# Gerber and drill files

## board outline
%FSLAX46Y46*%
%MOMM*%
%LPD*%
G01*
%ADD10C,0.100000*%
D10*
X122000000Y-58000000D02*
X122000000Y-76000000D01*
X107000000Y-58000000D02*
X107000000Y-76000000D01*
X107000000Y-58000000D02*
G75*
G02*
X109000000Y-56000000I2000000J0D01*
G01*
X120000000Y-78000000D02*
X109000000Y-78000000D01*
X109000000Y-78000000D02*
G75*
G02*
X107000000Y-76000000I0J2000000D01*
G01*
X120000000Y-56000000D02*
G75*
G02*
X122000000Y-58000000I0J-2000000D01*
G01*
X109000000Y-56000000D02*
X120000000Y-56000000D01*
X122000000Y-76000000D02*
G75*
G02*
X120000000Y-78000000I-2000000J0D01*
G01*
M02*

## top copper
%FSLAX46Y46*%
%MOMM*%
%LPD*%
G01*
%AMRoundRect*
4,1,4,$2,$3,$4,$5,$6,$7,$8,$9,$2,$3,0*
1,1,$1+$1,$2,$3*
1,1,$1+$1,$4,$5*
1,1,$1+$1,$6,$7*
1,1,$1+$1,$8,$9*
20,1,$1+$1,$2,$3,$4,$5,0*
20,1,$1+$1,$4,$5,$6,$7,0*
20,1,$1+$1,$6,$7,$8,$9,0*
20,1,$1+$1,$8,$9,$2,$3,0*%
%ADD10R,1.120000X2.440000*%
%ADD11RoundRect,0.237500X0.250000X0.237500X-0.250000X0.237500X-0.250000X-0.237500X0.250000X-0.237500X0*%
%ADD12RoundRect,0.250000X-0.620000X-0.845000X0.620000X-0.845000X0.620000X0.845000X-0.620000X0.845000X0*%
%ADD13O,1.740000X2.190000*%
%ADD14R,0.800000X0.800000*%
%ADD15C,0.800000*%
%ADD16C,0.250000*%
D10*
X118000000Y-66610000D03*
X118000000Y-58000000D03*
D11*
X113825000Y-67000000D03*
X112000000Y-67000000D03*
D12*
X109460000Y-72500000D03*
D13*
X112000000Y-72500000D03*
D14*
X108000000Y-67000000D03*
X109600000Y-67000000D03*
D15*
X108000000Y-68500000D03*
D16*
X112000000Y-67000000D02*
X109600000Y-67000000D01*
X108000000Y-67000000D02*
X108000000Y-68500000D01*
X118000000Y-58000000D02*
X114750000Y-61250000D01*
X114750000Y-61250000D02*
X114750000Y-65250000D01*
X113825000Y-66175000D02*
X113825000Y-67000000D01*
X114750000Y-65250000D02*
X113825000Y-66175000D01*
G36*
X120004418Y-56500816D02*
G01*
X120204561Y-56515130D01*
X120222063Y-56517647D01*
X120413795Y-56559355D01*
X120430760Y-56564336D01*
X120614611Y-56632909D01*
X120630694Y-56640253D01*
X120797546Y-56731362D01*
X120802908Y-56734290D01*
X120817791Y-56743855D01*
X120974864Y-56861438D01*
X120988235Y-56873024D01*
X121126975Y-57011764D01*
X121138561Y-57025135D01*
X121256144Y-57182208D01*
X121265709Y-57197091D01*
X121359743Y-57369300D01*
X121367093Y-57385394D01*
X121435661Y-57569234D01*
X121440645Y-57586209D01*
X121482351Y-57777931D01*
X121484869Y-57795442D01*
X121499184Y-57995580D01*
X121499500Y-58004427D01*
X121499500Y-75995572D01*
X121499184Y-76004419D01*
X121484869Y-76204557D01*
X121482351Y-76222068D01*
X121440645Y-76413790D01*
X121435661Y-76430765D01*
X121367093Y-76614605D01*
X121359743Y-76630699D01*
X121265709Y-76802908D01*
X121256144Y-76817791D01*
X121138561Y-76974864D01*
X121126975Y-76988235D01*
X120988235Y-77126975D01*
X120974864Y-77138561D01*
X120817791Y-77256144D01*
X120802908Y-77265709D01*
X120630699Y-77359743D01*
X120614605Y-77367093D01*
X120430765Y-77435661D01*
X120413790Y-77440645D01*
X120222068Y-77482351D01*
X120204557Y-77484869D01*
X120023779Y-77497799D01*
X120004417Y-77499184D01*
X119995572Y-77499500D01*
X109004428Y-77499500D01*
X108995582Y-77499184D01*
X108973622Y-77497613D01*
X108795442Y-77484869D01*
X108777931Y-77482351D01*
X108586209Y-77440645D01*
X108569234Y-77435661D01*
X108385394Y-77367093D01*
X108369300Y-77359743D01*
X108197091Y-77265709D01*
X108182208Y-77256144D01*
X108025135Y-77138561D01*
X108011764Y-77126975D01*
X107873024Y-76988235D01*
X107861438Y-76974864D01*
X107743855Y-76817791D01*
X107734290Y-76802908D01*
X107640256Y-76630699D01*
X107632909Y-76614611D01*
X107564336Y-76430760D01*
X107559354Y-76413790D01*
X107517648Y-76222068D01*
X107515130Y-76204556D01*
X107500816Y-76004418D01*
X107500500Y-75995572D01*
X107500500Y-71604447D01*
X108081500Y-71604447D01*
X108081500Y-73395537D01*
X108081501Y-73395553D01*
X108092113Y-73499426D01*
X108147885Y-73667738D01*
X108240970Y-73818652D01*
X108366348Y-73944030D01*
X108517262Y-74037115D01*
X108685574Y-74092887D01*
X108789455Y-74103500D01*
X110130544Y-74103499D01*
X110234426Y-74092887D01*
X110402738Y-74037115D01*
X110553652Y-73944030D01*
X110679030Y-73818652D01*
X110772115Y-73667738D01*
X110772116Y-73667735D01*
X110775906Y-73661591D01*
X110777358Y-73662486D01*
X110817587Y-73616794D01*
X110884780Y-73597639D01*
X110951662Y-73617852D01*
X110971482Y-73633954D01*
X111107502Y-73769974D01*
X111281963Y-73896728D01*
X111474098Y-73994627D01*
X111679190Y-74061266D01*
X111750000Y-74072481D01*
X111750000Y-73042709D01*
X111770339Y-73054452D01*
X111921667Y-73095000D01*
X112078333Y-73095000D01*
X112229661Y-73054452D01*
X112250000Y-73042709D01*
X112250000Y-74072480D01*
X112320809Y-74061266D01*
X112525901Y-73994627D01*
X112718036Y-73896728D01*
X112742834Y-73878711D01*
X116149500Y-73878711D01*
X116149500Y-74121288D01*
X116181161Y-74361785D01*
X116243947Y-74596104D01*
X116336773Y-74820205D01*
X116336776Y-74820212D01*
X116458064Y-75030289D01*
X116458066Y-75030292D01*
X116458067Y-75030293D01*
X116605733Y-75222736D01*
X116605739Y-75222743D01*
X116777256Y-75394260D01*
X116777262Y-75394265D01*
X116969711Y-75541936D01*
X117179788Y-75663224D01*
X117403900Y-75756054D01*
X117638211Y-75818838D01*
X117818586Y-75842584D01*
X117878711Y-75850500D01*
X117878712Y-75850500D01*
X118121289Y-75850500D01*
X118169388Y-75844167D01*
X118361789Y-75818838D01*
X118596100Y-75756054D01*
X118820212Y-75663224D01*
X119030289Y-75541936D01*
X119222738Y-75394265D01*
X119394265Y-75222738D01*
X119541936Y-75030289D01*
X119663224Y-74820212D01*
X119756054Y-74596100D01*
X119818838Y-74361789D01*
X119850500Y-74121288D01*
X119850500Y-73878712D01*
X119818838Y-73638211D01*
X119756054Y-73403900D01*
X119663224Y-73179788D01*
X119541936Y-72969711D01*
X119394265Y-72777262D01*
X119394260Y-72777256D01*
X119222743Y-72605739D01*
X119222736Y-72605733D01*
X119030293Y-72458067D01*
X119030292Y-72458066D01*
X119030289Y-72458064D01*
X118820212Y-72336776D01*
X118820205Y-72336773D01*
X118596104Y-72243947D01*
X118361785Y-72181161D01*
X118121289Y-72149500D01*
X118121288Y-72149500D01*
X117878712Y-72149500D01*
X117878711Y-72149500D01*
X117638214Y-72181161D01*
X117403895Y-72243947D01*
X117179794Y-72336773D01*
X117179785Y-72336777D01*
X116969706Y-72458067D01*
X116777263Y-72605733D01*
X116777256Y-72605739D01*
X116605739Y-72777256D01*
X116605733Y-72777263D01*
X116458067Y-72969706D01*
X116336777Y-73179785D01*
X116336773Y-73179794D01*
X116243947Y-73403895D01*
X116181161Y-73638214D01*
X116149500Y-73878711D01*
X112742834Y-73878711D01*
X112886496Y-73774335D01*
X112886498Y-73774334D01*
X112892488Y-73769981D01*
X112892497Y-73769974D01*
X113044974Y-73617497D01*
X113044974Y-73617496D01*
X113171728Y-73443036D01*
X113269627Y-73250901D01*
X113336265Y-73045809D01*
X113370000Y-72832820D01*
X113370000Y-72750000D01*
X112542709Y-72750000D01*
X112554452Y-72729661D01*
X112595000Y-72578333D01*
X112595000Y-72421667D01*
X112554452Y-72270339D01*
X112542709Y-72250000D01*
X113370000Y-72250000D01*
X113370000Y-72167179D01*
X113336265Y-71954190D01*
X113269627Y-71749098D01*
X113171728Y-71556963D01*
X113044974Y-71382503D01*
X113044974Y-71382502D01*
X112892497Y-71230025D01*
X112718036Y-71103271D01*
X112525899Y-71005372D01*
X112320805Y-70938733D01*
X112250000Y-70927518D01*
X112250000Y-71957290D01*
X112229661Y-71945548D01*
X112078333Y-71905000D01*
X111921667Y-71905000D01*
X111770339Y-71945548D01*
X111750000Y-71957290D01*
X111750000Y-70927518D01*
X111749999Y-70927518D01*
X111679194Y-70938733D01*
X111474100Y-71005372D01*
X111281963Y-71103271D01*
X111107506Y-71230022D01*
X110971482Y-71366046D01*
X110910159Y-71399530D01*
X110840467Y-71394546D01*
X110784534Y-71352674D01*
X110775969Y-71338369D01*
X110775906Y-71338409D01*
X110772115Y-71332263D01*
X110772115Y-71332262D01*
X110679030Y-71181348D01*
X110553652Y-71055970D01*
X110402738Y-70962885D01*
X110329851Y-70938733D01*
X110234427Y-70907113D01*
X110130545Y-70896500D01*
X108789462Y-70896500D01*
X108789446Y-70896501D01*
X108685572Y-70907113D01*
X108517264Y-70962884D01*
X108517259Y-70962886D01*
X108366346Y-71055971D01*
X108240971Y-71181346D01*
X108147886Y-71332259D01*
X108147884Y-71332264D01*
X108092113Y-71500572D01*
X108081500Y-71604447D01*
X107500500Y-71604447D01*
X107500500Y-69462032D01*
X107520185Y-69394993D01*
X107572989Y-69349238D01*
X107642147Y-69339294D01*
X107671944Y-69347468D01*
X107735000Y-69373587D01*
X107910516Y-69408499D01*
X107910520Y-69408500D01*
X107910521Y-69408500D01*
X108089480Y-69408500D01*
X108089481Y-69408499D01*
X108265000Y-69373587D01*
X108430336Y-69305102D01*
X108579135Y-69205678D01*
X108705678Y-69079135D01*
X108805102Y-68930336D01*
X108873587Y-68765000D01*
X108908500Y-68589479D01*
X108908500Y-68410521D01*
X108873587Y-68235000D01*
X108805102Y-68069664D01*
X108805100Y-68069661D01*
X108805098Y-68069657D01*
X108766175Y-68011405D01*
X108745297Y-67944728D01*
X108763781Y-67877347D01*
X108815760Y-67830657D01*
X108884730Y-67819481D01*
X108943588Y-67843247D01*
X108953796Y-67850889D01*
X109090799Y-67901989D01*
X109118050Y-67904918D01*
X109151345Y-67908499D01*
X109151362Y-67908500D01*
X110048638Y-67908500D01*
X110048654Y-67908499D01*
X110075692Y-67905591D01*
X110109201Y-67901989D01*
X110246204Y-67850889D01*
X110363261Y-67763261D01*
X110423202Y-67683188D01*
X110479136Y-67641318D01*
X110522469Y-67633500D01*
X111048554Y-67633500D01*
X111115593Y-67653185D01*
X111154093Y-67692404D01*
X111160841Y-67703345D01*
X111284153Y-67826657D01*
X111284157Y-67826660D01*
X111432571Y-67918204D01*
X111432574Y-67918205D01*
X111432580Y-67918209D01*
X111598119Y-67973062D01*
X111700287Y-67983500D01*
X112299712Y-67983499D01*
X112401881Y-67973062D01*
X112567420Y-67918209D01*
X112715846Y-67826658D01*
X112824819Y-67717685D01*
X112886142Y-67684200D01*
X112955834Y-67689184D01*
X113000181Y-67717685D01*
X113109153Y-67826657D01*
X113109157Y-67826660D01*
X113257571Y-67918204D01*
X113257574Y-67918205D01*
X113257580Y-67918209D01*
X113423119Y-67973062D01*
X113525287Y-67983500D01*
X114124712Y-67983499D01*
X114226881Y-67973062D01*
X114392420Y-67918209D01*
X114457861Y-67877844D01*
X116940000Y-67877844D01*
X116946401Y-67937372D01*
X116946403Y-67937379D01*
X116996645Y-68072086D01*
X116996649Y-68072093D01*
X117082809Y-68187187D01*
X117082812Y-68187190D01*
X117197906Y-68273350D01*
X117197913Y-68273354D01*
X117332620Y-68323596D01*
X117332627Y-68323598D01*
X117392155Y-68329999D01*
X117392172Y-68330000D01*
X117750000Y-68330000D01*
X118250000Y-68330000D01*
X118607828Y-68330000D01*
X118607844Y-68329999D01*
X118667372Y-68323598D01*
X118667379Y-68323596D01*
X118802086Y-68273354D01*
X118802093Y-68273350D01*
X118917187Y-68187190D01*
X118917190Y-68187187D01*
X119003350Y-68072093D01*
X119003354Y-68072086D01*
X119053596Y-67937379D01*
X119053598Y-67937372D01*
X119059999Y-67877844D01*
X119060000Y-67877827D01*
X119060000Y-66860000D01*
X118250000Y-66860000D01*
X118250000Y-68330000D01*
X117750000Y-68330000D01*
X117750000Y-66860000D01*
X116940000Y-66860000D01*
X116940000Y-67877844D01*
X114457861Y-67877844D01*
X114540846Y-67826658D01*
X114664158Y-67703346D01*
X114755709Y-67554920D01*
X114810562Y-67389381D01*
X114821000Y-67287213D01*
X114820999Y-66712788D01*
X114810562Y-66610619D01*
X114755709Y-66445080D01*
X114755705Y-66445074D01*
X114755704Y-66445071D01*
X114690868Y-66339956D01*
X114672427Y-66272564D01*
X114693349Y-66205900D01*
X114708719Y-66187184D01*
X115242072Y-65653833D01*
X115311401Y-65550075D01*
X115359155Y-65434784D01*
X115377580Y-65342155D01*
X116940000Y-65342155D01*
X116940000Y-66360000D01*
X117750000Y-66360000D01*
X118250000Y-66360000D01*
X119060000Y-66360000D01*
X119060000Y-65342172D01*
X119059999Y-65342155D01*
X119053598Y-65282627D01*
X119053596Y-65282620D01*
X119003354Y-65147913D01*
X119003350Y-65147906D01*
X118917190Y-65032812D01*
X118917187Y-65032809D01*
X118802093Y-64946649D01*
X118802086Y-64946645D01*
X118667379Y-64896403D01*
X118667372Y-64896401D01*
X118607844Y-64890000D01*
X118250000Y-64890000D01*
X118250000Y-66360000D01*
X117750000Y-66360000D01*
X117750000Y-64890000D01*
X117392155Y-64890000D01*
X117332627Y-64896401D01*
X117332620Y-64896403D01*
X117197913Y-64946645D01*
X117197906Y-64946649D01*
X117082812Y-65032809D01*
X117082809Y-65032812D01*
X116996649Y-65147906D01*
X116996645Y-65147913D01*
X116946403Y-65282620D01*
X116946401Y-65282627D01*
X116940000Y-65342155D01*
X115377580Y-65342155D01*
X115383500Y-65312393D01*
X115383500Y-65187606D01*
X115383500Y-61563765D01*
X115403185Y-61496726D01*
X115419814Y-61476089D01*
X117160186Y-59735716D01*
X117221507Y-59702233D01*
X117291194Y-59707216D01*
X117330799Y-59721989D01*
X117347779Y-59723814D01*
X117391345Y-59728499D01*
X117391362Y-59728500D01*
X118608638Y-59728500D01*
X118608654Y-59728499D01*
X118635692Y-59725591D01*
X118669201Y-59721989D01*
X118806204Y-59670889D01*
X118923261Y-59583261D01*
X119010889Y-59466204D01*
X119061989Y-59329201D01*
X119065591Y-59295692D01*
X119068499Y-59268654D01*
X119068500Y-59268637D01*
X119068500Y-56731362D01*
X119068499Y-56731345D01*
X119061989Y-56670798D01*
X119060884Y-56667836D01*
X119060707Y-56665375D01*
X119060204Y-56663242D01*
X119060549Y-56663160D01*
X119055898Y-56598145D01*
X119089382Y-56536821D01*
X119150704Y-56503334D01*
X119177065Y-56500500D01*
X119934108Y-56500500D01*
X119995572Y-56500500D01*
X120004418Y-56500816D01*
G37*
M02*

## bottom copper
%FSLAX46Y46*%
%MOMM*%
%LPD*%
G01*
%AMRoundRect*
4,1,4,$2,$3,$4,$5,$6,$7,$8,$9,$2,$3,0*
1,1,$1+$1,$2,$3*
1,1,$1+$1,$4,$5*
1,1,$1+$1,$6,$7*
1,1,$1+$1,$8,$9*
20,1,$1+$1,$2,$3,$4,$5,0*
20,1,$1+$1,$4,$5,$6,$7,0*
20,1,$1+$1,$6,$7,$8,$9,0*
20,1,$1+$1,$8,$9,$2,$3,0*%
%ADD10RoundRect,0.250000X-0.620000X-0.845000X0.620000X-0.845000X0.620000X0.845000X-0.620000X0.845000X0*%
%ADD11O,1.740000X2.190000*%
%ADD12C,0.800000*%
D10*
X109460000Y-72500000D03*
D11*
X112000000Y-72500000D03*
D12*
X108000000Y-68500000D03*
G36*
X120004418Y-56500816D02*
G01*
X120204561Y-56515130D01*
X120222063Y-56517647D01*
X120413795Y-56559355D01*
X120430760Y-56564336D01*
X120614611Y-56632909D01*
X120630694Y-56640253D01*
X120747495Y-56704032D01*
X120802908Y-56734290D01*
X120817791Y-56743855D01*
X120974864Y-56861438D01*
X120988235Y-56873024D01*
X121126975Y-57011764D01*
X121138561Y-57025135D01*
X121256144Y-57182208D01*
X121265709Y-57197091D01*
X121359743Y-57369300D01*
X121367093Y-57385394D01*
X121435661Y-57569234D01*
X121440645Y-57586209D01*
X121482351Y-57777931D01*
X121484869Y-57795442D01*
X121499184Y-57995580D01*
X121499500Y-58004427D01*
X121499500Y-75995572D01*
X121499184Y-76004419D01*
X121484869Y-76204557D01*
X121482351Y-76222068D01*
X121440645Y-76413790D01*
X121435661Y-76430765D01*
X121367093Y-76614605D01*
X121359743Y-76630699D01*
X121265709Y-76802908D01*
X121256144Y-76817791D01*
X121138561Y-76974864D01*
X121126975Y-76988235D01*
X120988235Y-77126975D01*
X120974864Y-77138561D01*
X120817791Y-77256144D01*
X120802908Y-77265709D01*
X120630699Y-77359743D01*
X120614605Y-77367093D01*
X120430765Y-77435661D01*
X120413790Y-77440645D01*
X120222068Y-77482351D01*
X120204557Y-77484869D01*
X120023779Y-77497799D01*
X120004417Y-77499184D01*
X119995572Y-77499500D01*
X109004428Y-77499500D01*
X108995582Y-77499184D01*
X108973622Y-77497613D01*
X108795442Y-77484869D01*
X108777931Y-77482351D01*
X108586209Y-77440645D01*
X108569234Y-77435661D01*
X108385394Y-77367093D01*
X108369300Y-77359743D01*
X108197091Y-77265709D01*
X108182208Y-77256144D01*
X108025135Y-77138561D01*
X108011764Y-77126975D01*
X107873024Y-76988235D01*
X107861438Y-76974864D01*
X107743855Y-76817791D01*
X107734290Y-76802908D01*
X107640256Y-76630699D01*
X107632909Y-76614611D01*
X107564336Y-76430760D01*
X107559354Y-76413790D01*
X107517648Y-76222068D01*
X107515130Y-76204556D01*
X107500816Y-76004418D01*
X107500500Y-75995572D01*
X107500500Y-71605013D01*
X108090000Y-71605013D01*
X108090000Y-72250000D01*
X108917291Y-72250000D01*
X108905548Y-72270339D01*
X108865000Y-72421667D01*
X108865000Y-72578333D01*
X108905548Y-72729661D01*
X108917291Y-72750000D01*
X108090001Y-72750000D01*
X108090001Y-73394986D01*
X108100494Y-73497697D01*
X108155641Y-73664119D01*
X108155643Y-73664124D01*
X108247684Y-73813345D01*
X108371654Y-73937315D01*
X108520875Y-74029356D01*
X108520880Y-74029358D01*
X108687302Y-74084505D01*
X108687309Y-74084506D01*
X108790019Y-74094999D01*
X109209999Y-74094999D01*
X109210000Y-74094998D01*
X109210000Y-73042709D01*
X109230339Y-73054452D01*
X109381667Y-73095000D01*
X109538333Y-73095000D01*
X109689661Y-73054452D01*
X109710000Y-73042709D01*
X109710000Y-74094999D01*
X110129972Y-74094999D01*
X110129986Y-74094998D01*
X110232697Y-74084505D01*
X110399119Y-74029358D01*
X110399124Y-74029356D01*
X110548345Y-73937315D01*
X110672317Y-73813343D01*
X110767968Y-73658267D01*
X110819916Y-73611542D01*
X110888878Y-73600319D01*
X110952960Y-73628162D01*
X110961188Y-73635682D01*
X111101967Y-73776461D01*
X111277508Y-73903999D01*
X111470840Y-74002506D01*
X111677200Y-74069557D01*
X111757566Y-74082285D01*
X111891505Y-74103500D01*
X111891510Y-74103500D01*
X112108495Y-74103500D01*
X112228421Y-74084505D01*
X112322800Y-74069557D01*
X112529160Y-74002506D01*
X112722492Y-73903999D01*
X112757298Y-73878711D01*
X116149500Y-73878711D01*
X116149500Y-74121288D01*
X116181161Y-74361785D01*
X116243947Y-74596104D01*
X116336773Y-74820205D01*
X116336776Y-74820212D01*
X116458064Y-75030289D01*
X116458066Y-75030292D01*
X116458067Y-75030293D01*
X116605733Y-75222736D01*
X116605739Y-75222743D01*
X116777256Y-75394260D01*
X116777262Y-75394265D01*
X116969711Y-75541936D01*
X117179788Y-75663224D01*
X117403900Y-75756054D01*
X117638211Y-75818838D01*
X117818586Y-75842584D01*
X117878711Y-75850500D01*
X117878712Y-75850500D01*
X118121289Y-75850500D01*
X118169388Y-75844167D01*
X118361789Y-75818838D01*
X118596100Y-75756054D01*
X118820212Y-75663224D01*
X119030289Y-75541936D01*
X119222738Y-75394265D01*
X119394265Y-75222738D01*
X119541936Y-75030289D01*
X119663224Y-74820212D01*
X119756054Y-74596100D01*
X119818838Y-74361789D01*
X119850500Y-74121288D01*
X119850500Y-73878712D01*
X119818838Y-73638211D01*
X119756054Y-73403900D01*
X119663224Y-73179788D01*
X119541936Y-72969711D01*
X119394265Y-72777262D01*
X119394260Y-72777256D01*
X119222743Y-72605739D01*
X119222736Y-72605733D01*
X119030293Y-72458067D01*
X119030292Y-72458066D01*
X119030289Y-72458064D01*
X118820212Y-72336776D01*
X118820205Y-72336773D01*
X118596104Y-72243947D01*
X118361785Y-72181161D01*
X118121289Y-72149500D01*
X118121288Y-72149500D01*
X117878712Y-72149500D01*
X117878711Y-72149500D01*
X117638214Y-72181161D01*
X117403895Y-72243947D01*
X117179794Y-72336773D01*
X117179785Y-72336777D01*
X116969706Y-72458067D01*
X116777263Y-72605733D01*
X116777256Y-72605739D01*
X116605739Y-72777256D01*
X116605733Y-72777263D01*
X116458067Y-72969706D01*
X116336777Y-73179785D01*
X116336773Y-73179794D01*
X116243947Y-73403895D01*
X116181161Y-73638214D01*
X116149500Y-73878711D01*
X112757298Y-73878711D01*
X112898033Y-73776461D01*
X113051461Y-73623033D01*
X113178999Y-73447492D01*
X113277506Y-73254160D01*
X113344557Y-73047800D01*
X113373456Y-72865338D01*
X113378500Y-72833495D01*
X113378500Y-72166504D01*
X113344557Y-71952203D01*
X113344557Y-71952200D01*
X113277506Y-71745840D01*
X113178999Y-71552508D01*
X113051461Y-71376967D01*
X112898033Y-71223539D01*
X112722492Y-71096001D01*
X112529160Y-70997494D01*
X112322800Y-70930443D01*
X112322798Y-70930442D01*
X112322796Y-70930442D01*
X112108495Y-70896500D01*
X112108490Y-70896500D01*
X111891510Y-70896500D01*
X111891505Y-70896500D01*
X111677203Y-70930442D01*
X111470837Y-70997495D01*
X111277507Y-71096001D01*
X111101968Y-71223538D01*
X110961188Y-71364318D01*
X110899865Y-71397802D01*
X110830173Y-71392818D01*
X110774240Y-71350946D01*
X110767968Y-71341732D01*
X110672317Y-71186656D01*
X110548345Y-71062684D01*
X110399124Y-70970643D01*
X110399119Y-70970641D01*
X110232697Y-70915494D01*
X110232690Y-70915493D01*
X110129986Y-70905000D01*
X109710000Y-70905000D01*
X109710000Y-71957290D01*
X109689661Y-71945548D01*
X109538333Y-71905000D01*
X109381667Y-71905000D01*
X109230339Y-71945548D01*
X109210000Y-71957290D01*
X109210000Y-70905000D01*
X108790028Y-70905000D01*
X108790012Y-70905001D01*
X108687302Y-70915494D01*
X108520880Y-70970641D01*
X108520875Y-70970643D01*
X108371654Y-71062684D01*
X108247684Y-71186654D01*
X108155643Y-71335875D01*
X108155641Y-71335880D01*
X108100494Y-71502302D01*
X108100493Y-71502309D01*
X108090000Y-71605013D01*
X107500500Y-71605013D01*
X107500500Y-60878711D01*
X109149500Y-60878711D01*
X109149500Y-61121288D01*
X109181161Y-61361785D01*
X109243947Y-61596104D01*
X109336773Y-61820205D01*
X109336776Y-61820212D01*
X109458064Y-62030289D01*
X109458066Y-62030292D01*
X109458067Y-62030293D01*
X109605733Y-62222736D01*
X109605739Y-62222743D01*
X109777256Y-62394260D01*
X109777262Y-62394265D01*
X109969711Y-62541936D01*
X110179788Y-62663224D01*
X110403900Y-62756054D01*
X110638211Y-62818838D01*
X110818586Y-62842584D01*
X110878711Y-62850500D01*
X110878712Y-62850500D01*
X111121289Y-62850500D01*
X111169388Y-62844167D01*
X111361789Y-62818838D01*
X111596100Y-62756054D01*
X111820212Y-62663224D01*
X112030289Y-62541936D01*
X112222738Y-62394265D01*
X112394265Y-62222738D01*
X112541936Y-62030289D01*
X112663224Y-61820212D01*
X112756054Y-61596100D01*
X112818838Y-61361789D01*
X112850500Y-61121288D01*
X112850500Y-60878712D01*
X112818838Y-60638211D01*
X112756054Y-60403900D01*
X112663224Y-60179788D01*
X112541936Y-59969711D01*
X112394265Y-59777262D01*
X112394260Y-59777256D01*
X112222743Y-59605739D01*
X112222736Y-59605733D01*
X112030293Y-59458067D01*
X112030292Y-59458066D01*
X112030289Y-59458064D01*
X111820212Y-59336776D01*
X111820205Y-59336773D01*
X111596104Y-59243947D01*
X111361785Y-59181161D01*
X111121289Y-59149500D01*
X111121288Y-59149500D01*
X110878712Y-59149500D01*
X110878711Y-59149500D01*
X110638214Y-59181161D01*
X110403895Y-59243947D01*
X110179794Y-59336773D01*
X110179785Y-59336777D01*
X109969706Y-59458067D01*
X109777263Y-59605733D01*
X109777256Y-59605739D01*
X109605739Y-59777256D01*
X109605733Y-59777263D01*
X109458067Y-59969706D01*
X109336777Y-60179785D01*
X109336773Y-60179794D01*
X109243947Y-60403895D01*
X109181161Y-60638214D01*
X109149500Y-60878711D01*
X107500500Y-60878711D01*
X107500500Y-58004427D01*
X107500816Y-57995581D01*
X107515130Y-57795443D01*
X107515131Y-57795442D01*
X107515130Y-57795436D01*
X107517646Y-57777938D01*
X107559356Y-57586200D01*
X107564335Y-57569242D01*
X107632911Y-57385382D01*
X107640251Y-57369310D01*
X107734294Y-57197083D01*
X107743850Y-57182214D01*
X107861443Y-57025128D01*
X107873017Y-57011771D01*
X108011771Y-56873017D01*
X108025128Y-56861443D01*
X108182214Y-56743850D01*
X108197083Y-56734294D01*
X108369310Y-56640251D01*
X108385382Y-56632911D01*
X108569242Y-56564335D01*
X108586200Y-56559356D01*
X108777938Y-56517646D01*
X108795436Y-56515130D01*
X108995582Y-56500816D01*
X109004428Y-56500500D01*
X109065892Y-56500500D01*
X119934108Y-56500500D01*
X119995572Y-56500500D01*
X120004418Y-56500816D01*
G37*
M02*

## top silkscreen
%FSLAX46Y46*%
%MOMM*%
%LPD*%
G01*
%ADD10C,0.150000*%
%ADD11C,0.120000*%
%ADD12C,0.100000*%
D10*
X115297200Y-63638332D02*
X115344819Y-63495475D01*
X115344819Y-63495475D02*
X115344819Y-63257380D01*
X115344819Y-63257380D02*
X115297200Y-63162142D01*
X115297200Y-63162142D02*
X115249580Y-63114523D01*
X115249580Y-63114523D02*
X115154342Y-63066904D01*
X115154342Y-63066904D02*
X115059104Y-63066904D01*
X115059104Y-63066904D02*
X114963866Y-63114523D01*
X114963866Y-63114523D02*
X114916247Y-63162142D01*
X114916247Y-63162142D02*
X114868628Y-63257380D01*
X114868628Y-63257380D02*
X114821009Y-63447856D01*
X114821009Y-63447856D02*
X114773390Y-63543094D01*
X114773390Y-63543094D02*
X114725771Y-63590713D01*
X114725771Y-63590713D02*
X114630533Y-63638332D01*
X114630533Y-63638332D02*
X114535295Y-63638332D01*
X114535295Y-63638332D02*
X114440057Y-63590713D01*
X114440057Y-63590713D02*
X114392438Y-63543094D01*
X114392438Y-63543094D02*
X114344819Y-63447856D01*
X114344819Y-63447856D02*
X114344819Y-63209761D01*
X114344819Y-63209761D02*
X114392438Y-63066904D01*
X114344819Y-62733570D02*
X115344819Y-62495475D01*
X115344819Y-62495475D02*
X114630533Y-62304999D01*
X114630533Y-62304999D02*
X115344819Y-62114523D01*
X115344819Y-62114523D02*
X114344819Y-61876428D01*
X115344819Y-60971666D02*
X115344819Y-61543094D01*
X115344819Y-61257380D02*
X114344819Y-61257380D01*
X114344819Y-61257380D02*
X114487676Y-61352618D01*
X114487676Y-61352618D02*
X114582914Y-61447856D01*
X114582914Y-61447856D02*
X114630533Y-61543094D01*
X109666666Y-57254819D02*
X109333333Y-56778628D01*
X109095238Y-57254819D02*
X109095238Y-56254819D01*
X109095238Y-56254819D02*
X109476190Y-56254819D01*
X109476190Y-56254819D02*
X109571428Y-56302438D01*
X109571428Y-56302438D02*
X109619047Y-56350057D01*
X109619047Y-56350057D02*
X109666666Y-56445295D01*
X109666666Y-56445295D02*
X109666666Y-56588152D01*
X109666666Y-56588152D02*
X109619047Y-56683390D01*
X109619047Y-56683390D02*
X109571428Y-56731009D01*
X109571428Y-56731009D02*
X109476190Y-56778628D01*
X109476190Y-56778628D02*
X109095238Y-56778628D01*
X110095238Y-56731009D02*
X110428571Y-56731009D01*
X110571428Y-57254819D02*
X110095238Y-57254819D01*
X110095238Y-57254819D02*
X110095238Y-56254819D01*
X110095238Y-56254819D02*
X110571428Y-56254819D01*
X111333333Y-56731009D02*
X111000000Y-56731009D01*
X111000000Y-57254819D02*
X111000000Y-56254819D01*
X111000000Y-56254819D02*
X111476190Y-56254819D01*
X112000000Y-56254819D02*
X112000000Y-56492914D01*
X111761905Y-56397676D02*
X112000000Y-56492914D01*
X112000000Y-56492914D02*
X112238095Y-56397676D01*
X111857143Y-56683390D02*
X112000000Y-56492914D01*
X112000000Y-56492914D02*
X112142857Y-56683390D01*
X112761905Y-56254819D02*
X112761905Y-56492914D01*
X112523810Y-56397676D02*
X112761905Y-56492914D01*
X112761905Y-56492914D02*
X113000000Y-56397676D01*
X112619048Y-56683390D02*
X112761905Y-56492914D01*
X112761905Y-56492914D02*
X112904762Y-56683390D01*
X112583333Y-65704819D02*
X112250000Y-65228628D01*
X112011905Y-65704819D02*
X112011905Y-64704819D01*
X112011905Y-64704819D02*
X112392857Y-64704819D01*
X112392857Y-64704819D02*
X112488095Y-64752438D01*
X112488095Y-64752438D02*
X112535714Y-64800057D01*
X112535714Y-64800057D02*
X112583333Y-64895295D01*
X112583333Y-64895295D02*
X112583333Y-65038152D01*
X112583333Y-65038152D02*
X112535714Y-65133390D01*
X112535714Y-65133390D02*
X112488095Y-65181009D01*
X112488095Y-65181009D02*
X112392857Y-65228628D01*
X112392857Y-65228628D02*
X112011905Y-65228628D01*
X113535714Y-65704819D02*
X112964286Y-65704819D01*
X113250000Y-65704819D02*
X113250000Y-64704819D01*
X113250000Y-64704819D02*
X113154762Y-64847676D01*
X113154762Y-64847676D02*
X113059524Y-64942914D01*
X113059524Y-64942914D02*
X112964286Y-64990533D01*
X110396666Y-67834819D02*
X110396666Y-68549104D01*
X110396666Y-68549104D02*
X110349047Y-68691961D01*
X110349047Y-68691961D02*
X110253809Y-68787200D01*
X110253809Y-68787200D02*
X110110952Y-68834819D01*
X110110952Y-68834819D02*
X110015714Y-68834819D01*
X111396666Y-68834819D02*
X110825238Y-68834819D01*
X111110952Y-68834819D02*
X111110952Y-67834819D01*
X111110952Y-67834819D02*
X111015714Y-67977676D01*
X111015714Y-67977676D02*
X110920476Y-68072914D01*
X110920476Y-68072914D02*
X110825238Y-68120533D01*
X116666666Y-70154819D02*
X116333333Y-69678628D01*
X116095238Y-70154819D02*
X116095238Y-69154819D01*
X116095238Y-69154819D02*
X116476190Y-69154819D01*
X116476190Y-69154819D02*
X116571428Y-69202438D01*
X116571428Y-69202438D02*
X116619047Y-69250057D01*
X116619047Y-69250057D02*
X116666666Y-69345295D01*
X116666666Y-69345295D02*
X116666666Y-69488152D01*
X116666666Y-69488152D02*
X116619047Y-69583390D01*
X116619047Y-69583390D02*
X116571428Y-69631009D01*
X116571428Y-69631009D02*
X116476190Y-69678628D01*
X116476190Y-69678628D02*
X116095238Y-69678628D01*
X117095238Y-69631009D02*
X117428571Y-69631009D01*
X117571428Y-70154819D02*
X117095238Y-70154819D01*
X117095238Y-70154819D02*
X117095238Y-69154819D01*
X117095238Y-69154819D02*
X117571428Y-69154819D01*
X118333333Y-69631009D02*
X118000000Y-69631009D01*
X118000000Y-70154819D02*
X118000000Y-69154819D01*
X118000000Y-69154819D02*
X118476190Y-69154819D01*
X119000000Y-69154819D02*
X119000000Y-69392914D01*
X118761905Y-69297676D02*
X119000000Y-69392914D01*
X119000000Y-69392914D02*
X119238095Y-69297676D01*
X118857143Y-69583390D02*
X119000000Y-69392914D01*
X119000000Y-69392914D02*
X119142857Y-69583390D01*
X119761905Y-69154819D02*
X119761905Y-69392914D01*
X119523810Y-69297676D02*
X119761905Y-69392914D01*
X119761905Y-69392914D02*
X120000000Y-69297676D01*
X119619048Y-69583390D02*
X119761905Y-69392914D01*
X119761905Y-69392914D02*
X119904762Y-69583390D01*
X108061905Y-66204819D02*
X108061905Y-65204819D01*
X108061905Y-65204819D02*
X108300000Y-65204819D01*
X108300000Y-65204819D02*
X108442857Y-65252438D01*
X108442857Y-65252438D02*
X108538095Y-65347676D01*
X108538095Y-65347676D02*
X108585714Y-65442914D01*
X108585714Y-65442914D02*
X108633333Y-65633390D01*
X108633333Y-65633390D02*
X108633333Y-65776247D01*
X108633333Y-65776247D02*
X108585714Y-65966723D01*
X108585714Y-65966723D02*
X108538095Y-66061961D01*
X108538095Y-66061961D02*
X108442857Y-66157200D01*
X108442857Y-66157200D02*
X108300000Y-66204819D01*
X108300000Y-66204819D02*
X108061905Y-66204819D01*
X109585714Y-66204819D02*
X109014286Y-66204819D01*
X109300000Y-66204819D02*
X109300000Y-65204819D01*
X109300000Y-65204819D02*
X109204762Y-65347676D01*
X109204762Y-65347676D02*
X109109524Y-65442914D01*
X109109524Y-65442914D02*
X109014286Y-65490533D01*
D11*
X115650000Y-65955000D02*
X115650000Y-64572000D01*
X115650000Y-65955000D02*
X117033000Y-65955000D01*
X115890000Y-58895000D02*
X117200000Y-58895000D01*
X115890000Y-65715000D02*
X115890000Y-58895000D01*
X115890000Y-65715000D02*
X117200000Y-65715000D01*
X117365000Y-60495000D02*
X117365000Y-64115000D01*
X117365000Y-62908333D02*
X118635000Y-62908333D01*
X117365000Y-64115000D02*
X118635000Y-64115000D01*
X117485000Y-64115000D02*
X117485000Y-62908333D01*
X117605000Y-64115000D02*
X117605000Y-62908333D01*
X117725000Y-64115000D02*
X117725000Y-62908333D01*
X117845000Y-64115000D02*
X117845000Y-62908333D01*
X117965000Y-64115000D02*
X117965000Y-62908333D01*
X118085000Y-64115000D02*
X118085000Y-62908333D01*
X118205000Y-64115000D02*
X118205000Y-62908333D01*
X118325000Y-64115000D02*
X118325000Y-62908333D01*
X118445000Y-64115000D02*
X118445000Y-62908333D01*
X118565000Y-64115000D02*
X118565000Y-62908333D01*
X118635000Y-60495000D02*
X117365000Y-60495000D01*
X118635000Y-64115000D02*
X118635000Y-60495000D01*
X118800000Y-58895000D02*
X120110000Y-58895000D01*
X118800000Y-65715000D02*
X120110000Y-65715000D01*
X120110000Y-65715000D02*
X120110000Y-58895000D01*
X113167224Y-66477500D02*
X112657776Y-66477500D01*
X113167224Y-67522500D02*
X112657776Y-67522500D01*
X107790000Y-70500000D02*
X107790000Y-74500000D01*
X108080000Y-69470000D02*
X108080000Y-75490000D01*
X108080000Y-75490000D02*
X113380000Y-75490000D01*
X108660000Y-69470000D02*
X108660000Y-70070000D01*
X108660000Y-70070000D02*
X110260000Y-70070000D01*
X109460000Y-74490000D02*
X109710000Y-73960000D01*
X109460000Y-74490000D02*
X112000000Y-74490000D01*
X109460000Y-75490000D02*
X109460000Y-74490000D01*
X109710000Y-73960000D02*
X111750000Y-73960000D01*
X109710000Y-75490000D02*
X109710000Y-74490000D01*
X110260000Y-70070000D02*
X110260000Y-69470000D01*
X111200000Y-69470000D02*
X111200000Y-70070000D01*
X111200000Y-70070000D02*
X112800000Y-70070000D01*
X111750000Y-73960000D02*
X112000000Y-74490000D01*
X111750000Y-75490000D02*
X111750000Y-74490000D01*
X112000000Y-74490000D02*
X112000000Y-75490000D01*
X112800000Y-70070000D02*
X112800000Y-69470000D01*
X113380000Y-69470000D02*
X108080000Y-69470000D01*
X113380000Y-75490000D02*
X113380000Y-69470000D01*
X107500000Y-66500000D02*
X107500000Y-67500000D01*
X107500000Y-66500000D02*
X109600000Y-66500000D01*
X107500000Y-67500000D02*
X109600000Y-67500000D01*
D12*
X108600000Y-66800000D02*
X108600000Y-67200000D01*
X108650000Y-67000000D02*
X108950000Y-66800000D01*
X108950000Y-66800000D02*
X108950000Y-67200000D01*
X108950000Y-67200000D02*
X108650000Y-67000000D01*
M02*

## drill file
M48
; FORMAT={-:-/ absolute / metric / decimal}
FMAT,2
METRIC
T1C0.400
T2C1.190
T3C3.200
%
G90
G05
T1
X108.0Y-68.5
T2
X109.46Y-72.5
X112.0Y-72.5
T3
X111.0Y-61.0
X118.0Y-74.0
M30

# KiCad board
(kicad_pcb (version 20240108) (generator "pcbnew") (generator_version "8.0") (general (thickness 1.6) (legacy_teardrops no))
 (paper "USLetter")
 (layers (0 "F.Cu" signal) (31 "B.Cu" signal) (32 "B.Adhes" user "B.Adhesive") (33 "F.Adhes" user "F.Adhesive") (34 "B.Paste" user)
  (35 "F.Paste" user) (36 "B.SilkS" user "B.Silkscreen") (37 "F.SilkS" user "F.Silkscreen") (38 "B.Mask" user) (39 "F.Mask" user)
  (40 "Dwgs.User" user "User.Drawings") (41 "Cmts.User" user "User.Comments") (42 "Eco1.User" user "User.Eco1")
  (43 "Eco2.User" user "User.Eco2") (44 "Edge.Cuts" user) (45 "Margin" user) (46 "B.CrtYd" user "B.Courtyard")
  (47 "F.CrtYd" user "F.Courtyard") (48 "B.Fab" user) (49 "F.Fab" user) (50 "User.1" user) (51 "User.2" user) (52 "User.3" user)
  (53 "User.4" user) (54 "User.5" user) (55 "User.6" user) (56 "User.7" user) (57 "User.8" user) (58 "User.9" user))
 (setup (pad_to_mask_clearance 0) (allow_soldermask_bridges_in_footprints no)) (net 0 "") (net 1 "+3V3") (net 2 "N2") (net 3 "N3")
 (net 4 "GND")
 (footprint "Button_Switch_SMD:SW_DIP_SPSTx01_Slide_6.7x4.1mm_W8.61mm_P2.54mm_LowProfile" (layer "F.Cu") (at 118 62.305 90)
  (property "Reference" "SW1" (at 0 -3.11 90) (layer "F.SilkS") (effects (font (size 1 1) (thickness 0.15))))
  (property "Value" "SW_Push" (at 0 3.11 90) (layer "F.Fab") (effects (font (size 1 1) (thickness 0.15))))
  (fp_line (start -3.65 -2.35) (end -2.267 -2.35) (stroke (width 0.12) (type solid)) (layer "F.SilkS"))
  (fp_line (start -3.65 -2.35) (end -3.65 -0.967) (stroke (width 0.12) (type solid)) (layer "F.SilkS"))
  (fp_line (start 3.41 -2.11) (end 3.41 -0.8) (stroke (width 0.12) (type solid)) (layer "F.SilkS"))
  (fp_line (start -3.41 -2.11) (end 3.41 -2.11) (stroke (width 0.12) (type solid)) (layer "F.SilkS"))
  (fp_line (start -3.41 -2.11) (end -3.41 -0.8) (stroke (width 0.12) (type solid)) (layer "F.SilkS"))
  (fp_line (start 1.81 -0.635) (end -1.81 -0.635) (stroke (width 0.12) (type solid)) (layer "F.SilkS"))
  (fp_line (start -0.603333 -0.635) (end -0.603333 0.635) (stroke (width 0.12) (type solid)) (layer "F.SilkS"))
  (fp_line (start -1.81 -0.635) (end -1.81 0.635) (stroke (width 0.12) (type solid)) (layer "F.SilkS"))
  (fp_line (start -1.81 -0.515) (end -0.603333 -0.515) (stroke (width 0.12) (type solid)) (layer "F.SilkS"))
  (fp_line (start -1.81 -0.395) (end -0.603333 -0.395) (stroke (width 0.12) (type solid)) (layer "F.SilkS"))
  (fp_line (start -1.81 -0.275) (end -0.603333 -0.275) (stroke (width 0.12) (type solid)) (layer "F.SilkS"))
  (fp_line (start -1.81 -0.155) (end -0.603333 -0.155) (stroke (width 0.12) (type solid)) (layer "F.SilkS"))
  (fp_line (start -1.81 -0.035) (end -0.603333 -0.035) (stroke (width 0.12) (type solid)) (layer "F.SilkS"))
  (fp_line (start -1.81 0.085) (end -0.603333 0.085) (stroke (width 0.12) (type solid)) (layer "F.SilkS"))
  (fp_line (start -1.81 0.205) (end -0.603333 0.205) (stroke (width 0.12) (type solid)) (layer "F.SilkS"))
  (fp_line (start -1.81 0.325) (end -0.603333 0.325) (stroke (width 0.12) (type solid)) (layer "F.SilkS"))
  (fp_line (start -1.81 0.445) (end -0.603333 0.445) (stroke (width 0.12) (type solid)) (layer "F.SilkS"))
  (fp_line (start -1.81 0.565) (end -0.603333 0.565) (stroke (width 0.12) (type solid)) (layer "F.SilkS"))
  (fp_line (start 1.81 0.635) (end 1.81 -0.635) (stroke (width 0.12) (type solid)) (layer "F.SilkS"))
  (fp_line (start -1.81 0.635) (end 1.81 0.635) (stroke (width 0.12) (type solid)) (layer "F.SilkS"))
  (fp_line (start 3.41 0.8) (end 3.41 2.11) (stroke (width 0.12) (type solid)) (layer "F.SilkS"))
  (fp_line (start -3.41 0.8) (end -3.41 2.11) (stroke (width 0.12) (type solid)) (layer "F.SilkS"))
  (fp_line (start -3.41 2.11) (end 3.41 2.11) (stroke (width 0.12) (type solid)) (layer "F.SilkS"))
  (pad "1" smd rect (at -4.305 0 90) (size 2.44 1.12) (layers "F.Cu" "F.Paste" "F.Mask") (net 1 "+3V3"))
  (pad "2" smd rect (at 4.305 0 90) (size 2.44 1.12) (layers "F.Cu" "F.Paste" "F.Mask") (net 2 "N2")))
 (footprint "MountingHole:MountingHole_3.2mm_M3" (layer "F.Cu") (at 111 61)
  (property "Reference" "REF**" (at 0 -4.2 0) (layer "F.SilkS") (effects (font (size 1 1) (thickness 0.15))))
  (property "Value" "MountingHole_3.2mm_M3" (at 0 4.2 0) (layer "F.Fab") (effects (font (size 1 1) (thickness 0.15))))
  (pad "" np_thru_hole circle (at 0 0) (size 3.2 3.2) (drill 3.2) (layers "*.Cu" "*.Mask")))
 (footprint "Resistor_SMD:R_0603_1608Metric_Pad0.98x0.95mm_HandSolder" (layer "F.Cu") (at 112.9125 67 180)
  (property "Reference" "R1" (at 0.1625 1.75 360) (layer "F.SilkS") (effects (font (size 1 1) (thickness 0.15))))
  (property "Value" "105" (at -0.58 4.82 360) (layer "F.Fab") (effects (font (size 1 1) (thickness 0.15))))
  (fp_line (start -0.254724 0.5225) (end 0.254724 0.5225) (stroke (width 0.12) (type solid)) (layer "F.SilkS"))
  (fp_line (start -0.254724 -0.5225) (end 0.254724 -0.5225) (stroke (width 0.12) (type solid)) (layer "F.SilkS"))
  (pad "1" smd roundrect (at -0.9125 0 180) (size 0.975 0.95) (layers "F.Cu" "F.Paste" "F.Mask") (roundrect_rratio 0.25) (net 2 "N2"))
  (pad "2" smd roundrect (at 0.9125 0 180) (size 0.975 0.95) (layers "F.Cu" "F.Paste" "F.Mask") (roundrect_rratio 0.25) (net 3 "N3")))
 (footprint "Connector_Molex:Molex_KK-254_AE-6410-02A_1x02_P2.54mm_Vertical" (layer "F.Cu") (at 109.46 72.5)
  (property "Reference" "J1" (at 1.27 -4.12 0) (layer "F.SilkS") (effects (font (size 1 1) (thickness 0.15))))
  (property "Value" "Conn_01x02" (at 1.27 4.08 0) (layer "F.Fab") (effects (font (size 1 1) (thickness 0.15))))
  (fp_line (start -1.67 -2) (end -1.67 2) (stroke (width 0.12) (type solid)) (layer "F.SilkS"))
  (fp_line (start -1.38 -3.03) (end -1.38 2.99) (stroke (width 0.12) (type solid)) (layer "F.SilkS"))
  (fp_line (start -1.38 2.99) (end 3.92 2.99) (stroke (width 0.12) (type solid)) (layer "F.SilkS"))
  (fp_line (start -0.8 -3.03) (end -0.8 -2.43) (stroke (width 0.12) (type solid)) (layer "F.SilkS"))
  (fp_line (start -0.8 -2.43) (end 0.8 -2.43) (stroke (width 0.12) (type solid)) (layer "F.SilkS"))
  (fp_line (start 0 1.99) (end 0.25 1.46) (stroke (width 0.12) (type solid)) (layer "F.SilkS"))
  (fp_line (start 0 1.99) (end 2.54 1.99) (stroke (width 0.12) (type solid)) (layer "F.SilkS"))
  (fp_line (start 0 2.99) (end 0 1.99) (stroke (width 0.12) (type solid)) (layer "F.SilkS"))
  (fp_line (start 0.25 1.46) (end 2.29 1.46) (stroke (width 0.12) (type solid)) (layer "F.SilkS"))
  (fp_line (start 0.25 2.99) (end 0.25 1.99) (stroke (width 0.12) (type solid)) (layer "F.SilkS"))
  (fp_line (start 0.8 -2.43) (end 0.8 -3.03) (stroke (width 0.12) (type solid)) (layer "F.SilkS"))
  (fp_line (start 1.74 -3.03) (end 1.74 -2.43) (stroke (width 0.12) (type solid)) (layer "F.SilkS"))
  (fp_line (start 1.74 -2.43) (end 3.34 -2.43) (stroke (width 0.12) (type solid)) (layer "F.SilkS"))
  (fp_line (start 2.29 1.46) (end 2.54 1.99) (stroke (width 0.12) (type solid)) (layer "F.SilkS"))
  (fp_line (start 2.29 2.99) (end 2.29 1.99) (stroke (width 0.12) (type solid)) (layer "F.SilkS"))
  (fp_line (start 2.54 1.99) (end 2.54 2.99) (stroke (width 0.12) (type solid)) (layer "F.SilkS"))
  (fp_line (start 3.34 -2.43) (end 3.34 -3.03) (stroke (width 0.12) (type solid)) (layer "F.SilkS"))
  (fp_line (start 3.92 -3.03) (end -1.38 -3.03) (stroke (width 0.12) (type solid)) (layer "F.SilkS"))
  (fp_line (start 3.92 2.99) (end 3.92 -3.03) (stroke (width 0.12) (type solid)) (layer "F.SilkS"))
  (pad "1" thru_hole roundrect (at 0 0) (size 1.74 2.19) (drill 1.19) (layers "*.Cu" "*.Mask") (remove_unused_layers no)
   (roundrect_rratio 0.143678) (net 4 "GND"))
  (pad "2" thru_hole oval (at 2.54 0) (size 1.74 2.19) (drill 1.19) (layers "*.Cu" "*.Mask") (remove_unused_layers no) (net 1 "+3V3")))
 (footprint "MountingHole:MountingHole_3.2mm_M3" (layer "F.Cu") (at 118 74)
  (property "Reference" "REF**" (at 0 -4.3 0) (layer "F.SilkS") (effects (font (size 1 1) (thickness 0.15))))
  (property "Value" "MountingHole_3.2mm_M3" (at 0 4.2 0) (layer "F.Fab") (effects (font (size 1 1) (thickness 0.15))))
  (pad "" np_thru_hole circle (at 0 0) (size 3.2 3.2) (drill 3.2) (layers "*.Cu" "*.Mask")))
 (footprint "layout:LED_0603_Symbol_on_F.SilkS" (layer "F.Cu") (at 108.8 67)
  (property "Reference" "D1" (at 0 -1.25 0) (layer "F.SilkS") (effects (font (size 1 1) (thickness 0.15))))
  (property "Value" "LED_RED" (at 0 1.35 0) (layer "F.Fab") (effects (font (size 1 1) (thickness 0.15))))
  (fp_line (start -1.3 -0.5) (end -1.3 0.5) (stroke (width 0.12) (type solid)) (layer "F.SilkS"))
  (fp_line (start -1.3 -0.5) (end 0.8 -0.5) (stroke (width 0.12) (type solid)) (layer "F.SilkS"))
  (fp_line (start -1.3 0.5) (end 0.8 0.5) (stroke (width 0.12) (type solid)) (layer "F.SilkS"))
  (fp_line (start -0.2 -0.2) (end -0.2 0.2) (stroke (width 0.1) (type solid)) (layer "F.SilkS"))
  (fp_line (start -0.15 0) (end 0.15 -0.2) (stroke (width 0.1) (type solid)) (layer "F.SilkS"))
  (fp_line (start 0.15 -0.2) (end 0.15 0.2) (stroke (width 0.1) (type solid)) (layer "F.SilkS"))
  (fp_line (start 0.15 0.2) (end -0.15 0) (stroke (width 0.1) (type solid)) (layer "F.SilkS"))
  (pad "1" smd rect (at -0.8 0 180) (size 0.8 0.8) (layers "F.Cu" "F.Paste" "F.Mask") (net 4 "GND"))
  (pad "2" smd rect (at 0.8 0 180) (size 0.8 0.8) (layers "F.Cu" "F.Paste" "F.Mask") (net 3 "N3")))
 (gr_line (start 122 58) (end 122 76) (stroke (width 0.1) (type default)) (layer "Edge.Cuts"))
 (gr_line (start 107 58) (end 107 76) (stroke (width 0.1) (type default)) (layer "Edge.Cuts"))
 (gr_arc (start 107 58) (mid 107.585786 56.585786) (end 109 56) (stroke (width 0.1) (type default)) (layer "Edge.Cuts"))
 (gr_line (start 120 78) (end 109 78) (stroke (width 0.1) (type default)) (layer "Edge.Cuts"))
 (gr_arc (start 109 78) (mid 107.585786 77.414214) (end 107 76) (stroke (width 0.1) (type default)) (layer "Edge.Cuts"))
 (gr_arc (start 120 56) (mid 121.414214 56.585786) (end 122 58) (stroke (width 0.1) (type default)) (layer "Edge.Cuts"))
 (gr_line (start 109 56) (end 120 56) (stroke (width 0.1) (type default)) (layer "Edge.Cuts"))
 (gr_arc (start 122 76) (mid 121.414214 77.414214) (end 120 78) (stroke (width 0.1) (type default)) (layer "Edge.Cuts"))
 (segment (start 112 67) (end 109.6 67) (width 0.25) (layer "F.Cu") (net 3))
 (segment (start 108 67) (end 108 68.5) (width 0.25) (layer "F.Cu") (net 4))
 (via (at 108 68.5) (size 0.8) (drill 0.4) (layers "F.Cu" "B.Cu") (free yes) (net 4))
 (segment (start 118 58) (end 114.75 61.25) (width 0.25) (layer "F.Cu") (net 2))
 (segment (start 114.75 61.25) (end 114.75 65.25) (width 0.25) (layer "F.Cu") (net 2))
 (segment (start 113.825 66.175) (end 113.825 67) (width 0.25) (layer "F.Cu") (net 2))
 (segment (start 114.75 65.25) (end 113.825 66.175) (width 0.25) (layer "F.Cu") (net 2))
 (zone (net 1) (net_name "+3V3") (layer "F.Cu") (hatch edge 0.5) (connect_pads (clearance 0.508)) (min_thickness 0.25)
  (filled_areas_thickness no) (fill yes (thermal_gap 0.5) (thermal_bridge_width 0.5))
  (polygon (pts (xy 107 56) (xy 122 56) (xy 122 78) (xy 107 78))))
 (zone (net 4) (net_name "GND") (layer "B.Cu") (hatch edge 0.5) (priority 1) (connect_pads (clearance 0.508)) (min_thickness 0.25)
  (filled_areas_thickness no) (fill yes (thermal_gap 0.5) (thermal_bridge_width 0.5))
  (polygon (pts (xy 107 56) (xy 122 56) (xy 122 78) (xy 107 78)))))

